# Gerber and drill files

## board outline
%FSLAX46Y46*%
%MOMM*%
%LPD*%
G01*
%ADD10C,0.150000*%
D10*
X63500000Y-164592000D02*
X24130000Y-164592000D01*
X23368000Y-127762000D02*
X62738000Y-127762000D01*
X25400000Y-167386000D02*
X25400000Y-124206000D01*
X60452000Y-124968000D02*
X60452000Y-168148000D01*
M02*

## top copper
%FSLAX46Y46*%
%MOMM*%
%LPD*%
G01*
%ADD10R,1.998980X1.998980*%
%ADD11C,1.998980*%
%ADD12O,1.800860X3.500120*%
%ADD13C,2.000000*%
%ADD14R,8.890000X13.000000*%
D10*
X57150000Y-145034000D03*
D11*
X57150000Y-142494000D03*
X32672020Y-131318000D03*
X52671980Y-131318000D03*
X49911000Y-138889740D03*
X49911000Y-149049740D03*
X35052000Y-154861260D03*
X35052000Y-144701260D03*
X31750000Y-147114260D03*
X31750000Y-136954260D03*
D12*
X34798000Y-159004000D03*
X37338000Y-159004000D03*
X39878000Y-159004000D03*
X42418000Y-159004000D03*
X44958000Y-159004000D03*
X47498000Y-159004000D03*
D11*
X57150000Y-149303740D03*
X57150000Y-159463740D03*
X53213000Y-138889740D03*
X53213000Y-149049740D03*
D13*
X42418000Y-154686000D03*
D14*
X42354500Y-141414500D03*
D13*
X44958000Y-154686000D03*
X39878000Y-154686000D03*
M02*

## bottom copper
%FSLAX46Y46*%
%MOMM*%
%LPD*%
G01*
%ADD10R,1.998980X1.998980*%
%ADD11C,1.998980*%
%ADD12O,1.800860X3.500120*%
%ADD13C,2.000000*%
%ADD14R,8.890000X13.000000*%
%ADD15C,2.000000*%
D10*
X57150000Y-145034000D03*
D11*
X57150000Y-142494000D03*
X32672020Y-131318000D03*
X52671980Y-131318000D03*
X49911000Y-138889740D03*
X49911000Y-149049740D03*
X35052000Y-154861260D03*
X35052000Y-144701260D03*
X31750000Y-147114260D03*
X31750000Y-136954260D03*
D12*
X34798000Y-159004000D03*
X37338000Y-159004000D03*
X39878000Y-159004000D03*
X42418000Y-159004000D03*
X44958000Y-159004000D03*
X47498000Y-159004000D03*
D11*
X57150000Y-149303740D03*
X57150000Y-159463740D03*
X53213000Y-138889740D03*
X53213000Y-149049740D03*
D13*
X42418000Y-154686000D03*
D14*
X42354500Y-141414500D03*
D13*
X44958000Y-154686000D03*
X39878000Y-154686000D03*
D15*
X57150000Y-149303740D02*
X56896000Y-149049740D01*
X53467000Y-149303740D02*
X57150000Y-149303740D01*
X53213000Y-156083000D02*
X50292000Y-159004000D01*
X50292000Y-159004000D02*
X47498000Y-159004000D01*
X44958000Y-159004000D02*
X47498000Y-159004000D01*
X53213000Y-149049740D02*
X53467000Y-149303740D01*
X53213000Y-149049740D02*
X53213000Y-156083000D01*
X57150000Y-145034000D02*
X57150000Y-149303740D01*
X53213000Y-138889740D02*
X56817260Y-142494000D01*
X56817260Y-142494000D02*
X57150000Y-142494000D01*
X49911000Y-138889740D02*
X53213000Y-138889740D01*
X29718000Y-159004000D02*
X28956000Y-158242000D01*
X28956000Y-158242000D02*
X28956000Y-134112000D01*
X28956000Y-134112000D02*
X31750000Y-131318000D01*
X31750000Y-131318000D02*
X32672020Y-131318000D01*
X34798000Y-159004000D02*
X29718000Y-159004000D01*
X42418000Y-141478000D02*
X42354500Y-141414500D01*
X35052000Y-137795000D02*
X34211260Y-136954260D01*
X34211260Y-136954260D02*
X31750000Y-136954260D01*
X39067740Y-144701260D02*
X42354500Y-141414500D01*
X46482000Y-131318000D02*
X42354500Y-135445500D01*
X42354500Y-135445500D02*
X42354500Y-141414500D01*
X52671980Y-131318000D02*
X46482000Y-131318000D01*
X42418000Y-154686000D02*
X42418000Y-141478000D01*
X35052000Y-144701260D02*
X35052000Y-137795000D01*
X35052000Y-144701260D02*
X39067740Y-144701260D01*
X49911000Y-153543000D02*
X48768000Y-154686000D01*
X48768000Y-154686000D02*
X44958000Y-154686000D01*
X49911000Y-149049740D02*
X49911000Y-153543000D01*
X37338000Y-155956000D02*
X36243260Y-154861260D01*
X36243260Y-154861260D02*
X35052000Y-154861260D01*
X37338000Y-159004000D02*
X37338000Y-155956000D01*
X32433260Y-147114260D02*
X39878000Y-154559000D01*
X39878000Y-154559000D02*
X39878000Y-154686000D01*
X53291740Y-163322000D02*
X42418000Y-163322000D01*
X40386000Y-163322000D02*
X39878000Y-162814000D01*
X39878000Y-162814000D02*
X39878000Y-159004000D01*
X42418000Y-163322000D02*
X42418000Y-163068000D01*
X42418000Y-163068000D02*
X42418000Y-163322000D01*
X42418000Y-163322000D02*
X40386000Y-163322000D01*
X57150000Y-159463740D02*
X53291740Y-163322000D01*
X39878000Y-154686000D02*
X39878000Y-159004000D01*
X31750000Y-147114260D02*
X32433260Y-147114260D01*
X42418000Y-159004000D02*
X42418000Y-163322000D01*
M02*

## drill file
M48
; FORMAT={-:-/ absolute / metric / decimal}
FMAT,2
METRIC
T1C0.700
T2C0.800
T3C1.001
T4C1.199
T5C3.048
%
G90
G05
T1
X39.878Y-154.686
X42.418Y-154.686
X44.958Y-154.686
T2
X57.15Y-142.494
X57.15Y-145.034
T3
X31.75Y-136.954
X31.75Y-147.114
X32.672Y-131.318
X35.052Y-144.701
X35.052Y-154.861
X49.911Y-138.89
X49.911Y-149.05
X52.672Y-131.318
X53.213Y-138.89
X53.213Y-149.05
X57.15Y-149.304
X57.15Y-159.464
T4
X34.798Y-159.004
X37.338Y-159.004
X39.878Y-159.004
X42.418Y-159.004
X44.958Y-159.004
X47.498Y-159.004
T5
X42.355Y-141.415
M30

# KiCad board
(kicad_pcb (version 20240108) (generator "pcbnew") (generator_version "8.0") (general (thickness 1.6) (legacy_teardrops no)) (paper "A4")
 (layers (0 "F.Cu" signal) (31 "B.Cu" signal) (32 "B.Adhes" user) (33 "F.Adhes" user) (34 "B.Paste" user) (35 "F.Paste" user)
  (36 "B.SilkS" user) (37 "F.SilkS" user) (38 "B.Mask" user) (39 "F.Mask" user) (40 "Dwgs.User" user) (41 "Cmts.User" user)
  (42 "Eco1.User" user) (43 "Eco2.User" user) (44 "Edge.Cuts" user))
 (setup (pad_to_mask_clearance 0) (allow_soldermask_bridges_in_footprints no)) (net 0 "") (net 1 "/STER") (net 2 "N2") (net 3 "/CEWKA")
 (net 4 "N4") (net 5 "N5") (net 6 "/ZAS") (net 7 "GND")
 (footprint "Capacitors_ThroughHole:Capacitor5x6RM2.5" (layer "F.Cu") (at 57.15 143.764)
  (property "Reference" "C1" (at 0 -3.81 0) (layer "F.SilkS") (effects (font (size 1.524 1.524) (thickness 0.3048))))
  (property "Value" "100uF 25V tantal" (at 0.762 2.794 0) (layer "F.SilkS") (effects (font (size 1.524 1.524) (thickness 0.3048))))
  (pad "1" thru_hole rect (at 0 1.27) (size 1.99898 1.99898) (drill 0.8001) (layers "*.Cu" "*.Mask" "F.SilkS") (remove_unused_layers no)
   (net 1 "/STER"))
  (pad "2" thru_hole circle (at 0 -1.27) (size 1.99898 1.99898) (drill 0.8001) (layers "*.Cu" "*.Mask" "F.SilkS") (remove_unused_layers no)
   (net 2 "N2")))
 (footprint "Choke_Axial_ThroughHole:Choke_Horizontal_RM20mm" (layer "F.Cu") (at 42.672 131.318)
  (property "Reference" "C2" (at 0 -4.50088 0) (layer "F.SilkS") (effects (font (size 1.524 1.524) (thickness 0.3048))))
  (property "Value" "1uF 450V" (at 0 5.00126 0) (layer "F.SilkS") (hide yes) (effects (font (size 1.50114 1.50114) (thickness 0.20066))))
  (pad "1" thru_hole circle (at -9.99998 0) (size 1.99898 1.99898) (drill 1.00076) (layers "*.Cu") (remove_unused_layers no)
   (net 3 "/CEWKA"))
  (pad "2" thru_hole circle (at 9.99998 0) (size 1.99898 1.99898) (drill 1.00076) (layers "*.Cu") (remove_unused_layers no) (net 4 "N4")))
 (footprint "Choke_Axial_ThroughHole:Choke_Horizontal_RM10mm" (layer "F.Cu") (at 49.911 143.891 -90)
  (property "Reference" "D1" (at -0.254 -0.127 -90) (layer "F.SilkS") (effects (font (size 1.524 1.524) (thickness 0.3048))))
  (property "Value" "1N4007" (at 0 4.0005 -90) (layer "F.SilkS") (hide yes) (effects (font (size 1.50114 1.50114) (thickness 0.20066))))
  (pad "1" thru_hole circle (at -5.00126 0 270) (size 1.99898 1.99898) (drill 1.00076) (layers "*.Cu") (remove_unused_layers no)
   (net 2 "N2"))
  (pad "2" thru_hole circle (at 5.15874 0 270) (size 1.99898 1.99898) (drill 1.00076) (layers "*.Cu") (remove_unused_layers no) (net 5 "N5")))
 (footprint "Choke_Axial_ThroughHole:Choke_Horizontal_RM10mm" (layer "F.Cu") (at 35.052 149.86 90)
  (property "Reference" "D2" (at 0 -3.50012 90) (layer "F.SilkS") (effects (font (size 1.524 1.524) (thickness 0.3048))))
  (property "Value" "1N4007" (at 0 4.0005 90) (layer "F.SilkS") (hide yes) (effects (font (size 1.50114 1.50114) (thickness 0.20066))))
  (pad "1" thru_hole circle (at -5.00126 0 90) (size 1.99898 1.99898) (drill 1.00076) (layers "*.Cu") (remove_unused_layers no)
   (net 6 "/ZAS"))
  (pad "2" thru_hole circle (at 5.15874 0 90) (size 1.99898 1.99898) (drill 1.00076) (layers "*.Cu") (remove_unused_layers no) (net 4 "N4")))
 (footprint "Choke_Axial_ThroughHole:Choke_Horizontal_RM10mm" (layer "F.Cu") (at 31.75 142.113 90)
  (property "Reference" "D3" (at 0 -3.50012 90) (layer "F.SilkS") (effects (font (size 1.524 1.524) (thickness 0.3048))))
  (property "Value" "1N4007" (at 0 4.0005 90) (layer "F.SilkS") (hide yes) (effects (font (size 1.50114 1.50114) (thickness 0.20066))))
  (pad "1" thru_hole circle (at -5.00126 0 90) (size 1.99898 1.99898) (drill 1.00076) (layers "*.Cu") (remove_unused_layers no)
   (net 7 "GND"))
  (pad "2" thru_hole circle (at 5.15874 0 90) (size 1.99898 1.99898) (drill 1.00076) (layers "*.Cu") (remove_unused_layers no) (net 4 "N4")))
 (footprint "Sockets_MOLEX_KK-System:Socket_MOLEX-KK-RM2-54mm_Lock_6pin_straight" (layer "F.Cu") (at 41.148 159.004)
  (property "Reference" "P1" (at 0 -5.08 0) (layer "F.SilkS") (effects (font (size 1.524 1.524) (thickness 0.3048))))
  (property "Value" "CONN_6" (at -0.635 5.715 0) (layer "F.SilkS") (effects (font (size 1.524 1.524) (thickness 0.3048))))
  (pad "1" thru_hole oval (at -6.35 0) (size 1.80086 3.50012) (drill 1.19888) (layers "*.Cu" "*.Mask" "F.SilkS") (remove_unused_layers no)
   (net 3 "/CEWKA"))
  (pad "2" thru_hole oval (at -3.81 0) (size 1.80086 3.50012) (drill 1.19888) (layers "*.Cu" "*.Mask" "F.SilkS") (remove_unused_layers no)
   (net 6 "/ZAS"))
  (pad "3" thru_hole oval (at -1.27 0) (size 1.80086 3.50012) (drill 1.19888) (layers "*.Cu" "*.Mask" "F.SilkS") (remove_unused_layers no)
   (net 7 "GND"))
  (pad "4" thru_hole oval (at 1.27 0) (size 1.80086 3.50012) (drill 1.19888) (layers "*.Cu" "*.Mask" "F.SilkS") (remove_unused_layers no)
   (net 7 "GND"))
  (pad "5" thru_hole oval (at 3.81 0) (size 1.80086 3.50012) (drill 1.19888) (layers "*.Cu" "*.Mask" "F.SilkS") (remove_unused_layers no)
   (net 1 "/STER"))
  (pad "6" thru_hole oval (at 6.35 0) (size 1.80086 3.50012) (drill 1.19888) (layers "*.Cu" "*.Mask" "F.SilkS") (remove_unused_layers no)
   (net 1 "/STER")))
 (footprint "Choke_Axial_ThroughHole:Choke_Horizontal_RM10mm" (layer "F.Cu") (at 57.15 154.305 -90)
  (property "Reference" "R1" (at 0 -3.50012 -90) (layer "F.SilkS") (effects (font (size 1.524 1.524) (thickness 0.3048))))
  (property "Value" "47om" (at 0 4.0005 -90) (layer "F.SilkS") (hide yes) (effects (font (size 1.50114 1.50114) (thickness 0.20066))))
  (pad "1" thru_hole circle (at -5.00126 0 270) (size 1.99898 1.99898) (drill 1.00076) (layers "*.Cu") (remove_unused_layers no)
   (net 1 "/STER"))
  (pad "2" thru_hole circle (at 5.15874 0 270) (size 1.99898 1.99898) (drill 1.00076) (layers "*.Cu") (remove_unused_layers no)
   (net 7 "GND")))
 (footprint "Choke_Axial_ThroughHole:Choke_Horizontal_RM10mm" (layer "F.Cu") (at 53.213 143.891 -90)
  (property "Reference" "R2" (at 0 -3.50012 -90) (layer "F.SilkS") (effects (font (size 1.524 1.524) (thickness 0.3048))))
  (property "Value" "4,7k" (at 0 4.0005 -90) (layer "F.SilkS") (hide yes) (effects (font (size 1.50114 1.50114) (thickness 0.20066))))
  (pad "1" thru_hole circle (at -5.00126 0 270) (size 1.99898 1.99898) (drill 1.00076) (layers "*.Cu") (remove_unused_layers no)
   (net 2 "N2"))
  (pad "2" thru_hole circle (at 5.15874 0 270) (size 1.99898 1.99898) (drill 1.00076) (layers "*.Cu") (remove_unused_layers no)
   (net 1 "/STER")))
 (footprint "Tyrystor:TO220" (layer "F.Cu") (at 42.418 154.686 90)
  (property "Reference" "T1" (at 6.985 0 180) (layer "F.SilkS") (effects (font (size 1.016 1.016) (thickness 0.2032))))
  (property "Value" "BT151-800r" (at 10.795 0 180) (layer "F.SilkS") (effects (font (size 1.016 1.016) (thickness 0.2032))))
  (pad "A" thru_hole circle (at 0 0 90) (size 2 2) (drill 0.7) (layers "*.Cu" "*.Mask" "F.SilkS") (remove_unused_layers no) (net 4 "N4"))
  (pad "A" thru_hole rect (at 13.2715 -0.0635 90) (size 13 8.89) (drill 3.048) (layers "*.Cu" "*.SilkS" "*.Mask") (remove_unused_layers no)
   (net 4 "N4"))
  (pad "G" thru_hole circle (at 0 2.54 90) (size 2 2) (drill 0.7) (layers "*.Cu" "*.Mask" "F.SilkS") (remove_unused_layers no) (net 5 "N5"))
  (pad "K" thru_hole circle (at 0 -2.54 90) (size 2 2) (drill 0.7) (layers "*.Cu" "*.Mask" "F.SilkS") (remove_unused_layers no)
   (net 7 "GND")))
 (gr_line (start 63.5 164.592) (end 24.13 164.592) (stroke (width 0.15) (type solid)) (layer "Edge.Cuts"))
 (gr_line (start 23.368 127.762) (end 62.738 127.762) (stroke (width 0.15) (type solid)) (layer "Edge.Cuts"))
 (gr_line (start 25.4 167.386) (end 25.4 124.206) (stroke (width 0.15) (type solid)) (layer "Edge.Cuts"))
 (gr_line (start 60.452 124.968) (end 60.452 168.148) (stroke (width 0.15) (type solid)) (layer "Edge.Cuts"))
 (segment (start 57.15 149.30374) (end 56.896 149.04974) (width 2) (layer "B.Cu") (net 1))
 (segment (start 53.467 149.30374) (end 57.15 149.30374) (width 2) (layer "B.Cu") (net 1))
 (segment (start 53.213 156.083) (end 50.292 159.004) (width 2) (layer "B.Cu") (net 1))
 (segment (start 50.292 159.004) (end 47.498 159.004) (width 2) (layer "B.Cu") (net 1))
 (segment (start 44.958 159.004) (end 47.498 159.004) (width 2) (layer "B.Cu") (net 1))
 (segment (start 53.213 149.04974) (end 53.467 149.30374) (width 2) (layer "B.Cu") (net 1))
 (segment (start 53.213 149.04974) (end 53.213 156.083) (width 2) (layer "B.Cu") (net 1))
 (segment (start 57.15 145.034) (end 57.15 149.30374) (width 2) (layer "B.Cu") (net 1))
 (segment (start 53.213 138.88974) (end 56.81726 142.494) (width 2) (layer "B.Cu") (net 2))
 (segment (start 56.81726 142.494) (end 57.15 142.494) (width 2) (layer "B.Cu") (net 2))
 (segment (start 49.911 138.88974) (end 53.213 138.88974) (width 2) (layer "B.Cu") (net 2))
 (segment (start 29.718 159.004) (end 28.956 158.242) (width 2) (layer "B.Cu") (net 3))
 (segment (start 28.956 158.242) (end 28.956 134.112) (width 2) (layer "B.Cu") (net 3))
 (segment (start 28.956 134.112) (end 31.75 131.318) (width 2) (layer "B.Cu") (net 3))
 (segment (start 31.75 131.318) (end 32.67202 131.318) (width 2) (layer "B.Cu") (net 3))
 (segment (start 34.798 159.004) (end 29.718 159.004) (width 2) (layer "B.Cu") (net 3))
 (segment (start 42.418 141.478) (end 42.3545 141.4145) (width 2) (layer "B.Cu") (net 4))
 (segment (start 35.052 137.795) (end 34.21126 136.95426) (width 2) (layer "B.Cu") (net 4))
 (segment (start 34.21126 136.95426) (end 31.75 136.95426) (width 2) (layer "B.Cu") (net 4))
 (segment (start 39.06774 144.70126) (end 42.3545 141.4145) (width 2) (layer "B.Cu") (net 4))
 (segment (start 46.482 131.318) (end 42.3545 135.4455) (width 2) (layer "B.Cu") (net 4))
 (segment (start 42.3545 135.4455) (end 42.3545 141.4145) (width 2) (layer "B.Cu") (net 4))
 (segment (start 52.67198 131.318) (end 46.482 131.318) (width 2) (layer "B.Cu") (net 4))
 (segment (start 42.418 154.686) (end 42.418 141.478) (width 2) (layer "B.Cu") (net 4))
 (segment (start 35.052 144.70126) (end 35.052 137.795) (width 2) (layer "B.Cu") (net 4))
 (segment (start 35.052 144.70126) (end 39.06774 144.70126) (width 2) (layer "B.Cu") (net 4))
 (segment (start 49.911 153.543) (end 48.768 154.686) (width 2) (layer "B.Cu") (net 5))
 (segment (start 48.768 154.686) (end 44.958 154.686) (width 2) (layer "B.Cu") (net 5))
 (segment (start 49.911 149.04974) (end 49.911 153.543) (width 2) (layer "B.Cu") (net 5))
 (segment (start 37.338 155.956) (end 36.24326 154.86126) (width 2) (layer "B.Cu") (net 6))
 (segment (start 36.24326 154.86126) (end 35.052 154.86126) (width 2) (layer "B.Cu") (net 6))
 (segment (start 37.338 159.004) (end 37.338 155.956) (width 2) (layer "B.Cu") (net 6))
 (segment (start 32.43326 147.11426) (end 39.878 154.559) (width 2) (layer "B.Cu") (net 7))
 (segment (start 39.878 154.559) (end 39.878 154.686) (width 2) (layer "B.Cu") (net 7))
 (segment (start 53.29174 163.322) (end 42.418 163.322) (width 2) (layer "B.Cu") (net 7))
 (segment (start 40.386 163.322) (end 39.878 162.814) (width 2) (layer "B.Cu") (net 7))
 (segment (start 39.878 162.814) (end 39.878 159.004) (width 2) (layer "B.Cu") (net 7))
 (segment (start 42.418 163.322) (end 42.418 163.068) (width 2) (layer "B.Cu") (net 7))
 (segment (start 42.418 163.068) (end 42.418 163.322) (width 2) (layer "B.Cu") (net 7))
 (segment (start 42.418 163.322) (end 40.386 163.322) (width 2) (layer "B.Cu") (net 7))
 (segment (start 57.15 159.46374) (end 53.29174 163.322) (width 2) (layer "B.Cu") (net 7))
 (segment (start 39.878 154.686) (end 39.878 159.004) (width 2) (layer "B.Cu") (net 7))
 (segment (start 31.75 147.11426) (end 32.43326 147.11426) (width 2) (layer "B.Cu") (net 7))
 (segment (start 42.418 159.004) (end 42.418 163.322) (width 2) (layer "B.Cu") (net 7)))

